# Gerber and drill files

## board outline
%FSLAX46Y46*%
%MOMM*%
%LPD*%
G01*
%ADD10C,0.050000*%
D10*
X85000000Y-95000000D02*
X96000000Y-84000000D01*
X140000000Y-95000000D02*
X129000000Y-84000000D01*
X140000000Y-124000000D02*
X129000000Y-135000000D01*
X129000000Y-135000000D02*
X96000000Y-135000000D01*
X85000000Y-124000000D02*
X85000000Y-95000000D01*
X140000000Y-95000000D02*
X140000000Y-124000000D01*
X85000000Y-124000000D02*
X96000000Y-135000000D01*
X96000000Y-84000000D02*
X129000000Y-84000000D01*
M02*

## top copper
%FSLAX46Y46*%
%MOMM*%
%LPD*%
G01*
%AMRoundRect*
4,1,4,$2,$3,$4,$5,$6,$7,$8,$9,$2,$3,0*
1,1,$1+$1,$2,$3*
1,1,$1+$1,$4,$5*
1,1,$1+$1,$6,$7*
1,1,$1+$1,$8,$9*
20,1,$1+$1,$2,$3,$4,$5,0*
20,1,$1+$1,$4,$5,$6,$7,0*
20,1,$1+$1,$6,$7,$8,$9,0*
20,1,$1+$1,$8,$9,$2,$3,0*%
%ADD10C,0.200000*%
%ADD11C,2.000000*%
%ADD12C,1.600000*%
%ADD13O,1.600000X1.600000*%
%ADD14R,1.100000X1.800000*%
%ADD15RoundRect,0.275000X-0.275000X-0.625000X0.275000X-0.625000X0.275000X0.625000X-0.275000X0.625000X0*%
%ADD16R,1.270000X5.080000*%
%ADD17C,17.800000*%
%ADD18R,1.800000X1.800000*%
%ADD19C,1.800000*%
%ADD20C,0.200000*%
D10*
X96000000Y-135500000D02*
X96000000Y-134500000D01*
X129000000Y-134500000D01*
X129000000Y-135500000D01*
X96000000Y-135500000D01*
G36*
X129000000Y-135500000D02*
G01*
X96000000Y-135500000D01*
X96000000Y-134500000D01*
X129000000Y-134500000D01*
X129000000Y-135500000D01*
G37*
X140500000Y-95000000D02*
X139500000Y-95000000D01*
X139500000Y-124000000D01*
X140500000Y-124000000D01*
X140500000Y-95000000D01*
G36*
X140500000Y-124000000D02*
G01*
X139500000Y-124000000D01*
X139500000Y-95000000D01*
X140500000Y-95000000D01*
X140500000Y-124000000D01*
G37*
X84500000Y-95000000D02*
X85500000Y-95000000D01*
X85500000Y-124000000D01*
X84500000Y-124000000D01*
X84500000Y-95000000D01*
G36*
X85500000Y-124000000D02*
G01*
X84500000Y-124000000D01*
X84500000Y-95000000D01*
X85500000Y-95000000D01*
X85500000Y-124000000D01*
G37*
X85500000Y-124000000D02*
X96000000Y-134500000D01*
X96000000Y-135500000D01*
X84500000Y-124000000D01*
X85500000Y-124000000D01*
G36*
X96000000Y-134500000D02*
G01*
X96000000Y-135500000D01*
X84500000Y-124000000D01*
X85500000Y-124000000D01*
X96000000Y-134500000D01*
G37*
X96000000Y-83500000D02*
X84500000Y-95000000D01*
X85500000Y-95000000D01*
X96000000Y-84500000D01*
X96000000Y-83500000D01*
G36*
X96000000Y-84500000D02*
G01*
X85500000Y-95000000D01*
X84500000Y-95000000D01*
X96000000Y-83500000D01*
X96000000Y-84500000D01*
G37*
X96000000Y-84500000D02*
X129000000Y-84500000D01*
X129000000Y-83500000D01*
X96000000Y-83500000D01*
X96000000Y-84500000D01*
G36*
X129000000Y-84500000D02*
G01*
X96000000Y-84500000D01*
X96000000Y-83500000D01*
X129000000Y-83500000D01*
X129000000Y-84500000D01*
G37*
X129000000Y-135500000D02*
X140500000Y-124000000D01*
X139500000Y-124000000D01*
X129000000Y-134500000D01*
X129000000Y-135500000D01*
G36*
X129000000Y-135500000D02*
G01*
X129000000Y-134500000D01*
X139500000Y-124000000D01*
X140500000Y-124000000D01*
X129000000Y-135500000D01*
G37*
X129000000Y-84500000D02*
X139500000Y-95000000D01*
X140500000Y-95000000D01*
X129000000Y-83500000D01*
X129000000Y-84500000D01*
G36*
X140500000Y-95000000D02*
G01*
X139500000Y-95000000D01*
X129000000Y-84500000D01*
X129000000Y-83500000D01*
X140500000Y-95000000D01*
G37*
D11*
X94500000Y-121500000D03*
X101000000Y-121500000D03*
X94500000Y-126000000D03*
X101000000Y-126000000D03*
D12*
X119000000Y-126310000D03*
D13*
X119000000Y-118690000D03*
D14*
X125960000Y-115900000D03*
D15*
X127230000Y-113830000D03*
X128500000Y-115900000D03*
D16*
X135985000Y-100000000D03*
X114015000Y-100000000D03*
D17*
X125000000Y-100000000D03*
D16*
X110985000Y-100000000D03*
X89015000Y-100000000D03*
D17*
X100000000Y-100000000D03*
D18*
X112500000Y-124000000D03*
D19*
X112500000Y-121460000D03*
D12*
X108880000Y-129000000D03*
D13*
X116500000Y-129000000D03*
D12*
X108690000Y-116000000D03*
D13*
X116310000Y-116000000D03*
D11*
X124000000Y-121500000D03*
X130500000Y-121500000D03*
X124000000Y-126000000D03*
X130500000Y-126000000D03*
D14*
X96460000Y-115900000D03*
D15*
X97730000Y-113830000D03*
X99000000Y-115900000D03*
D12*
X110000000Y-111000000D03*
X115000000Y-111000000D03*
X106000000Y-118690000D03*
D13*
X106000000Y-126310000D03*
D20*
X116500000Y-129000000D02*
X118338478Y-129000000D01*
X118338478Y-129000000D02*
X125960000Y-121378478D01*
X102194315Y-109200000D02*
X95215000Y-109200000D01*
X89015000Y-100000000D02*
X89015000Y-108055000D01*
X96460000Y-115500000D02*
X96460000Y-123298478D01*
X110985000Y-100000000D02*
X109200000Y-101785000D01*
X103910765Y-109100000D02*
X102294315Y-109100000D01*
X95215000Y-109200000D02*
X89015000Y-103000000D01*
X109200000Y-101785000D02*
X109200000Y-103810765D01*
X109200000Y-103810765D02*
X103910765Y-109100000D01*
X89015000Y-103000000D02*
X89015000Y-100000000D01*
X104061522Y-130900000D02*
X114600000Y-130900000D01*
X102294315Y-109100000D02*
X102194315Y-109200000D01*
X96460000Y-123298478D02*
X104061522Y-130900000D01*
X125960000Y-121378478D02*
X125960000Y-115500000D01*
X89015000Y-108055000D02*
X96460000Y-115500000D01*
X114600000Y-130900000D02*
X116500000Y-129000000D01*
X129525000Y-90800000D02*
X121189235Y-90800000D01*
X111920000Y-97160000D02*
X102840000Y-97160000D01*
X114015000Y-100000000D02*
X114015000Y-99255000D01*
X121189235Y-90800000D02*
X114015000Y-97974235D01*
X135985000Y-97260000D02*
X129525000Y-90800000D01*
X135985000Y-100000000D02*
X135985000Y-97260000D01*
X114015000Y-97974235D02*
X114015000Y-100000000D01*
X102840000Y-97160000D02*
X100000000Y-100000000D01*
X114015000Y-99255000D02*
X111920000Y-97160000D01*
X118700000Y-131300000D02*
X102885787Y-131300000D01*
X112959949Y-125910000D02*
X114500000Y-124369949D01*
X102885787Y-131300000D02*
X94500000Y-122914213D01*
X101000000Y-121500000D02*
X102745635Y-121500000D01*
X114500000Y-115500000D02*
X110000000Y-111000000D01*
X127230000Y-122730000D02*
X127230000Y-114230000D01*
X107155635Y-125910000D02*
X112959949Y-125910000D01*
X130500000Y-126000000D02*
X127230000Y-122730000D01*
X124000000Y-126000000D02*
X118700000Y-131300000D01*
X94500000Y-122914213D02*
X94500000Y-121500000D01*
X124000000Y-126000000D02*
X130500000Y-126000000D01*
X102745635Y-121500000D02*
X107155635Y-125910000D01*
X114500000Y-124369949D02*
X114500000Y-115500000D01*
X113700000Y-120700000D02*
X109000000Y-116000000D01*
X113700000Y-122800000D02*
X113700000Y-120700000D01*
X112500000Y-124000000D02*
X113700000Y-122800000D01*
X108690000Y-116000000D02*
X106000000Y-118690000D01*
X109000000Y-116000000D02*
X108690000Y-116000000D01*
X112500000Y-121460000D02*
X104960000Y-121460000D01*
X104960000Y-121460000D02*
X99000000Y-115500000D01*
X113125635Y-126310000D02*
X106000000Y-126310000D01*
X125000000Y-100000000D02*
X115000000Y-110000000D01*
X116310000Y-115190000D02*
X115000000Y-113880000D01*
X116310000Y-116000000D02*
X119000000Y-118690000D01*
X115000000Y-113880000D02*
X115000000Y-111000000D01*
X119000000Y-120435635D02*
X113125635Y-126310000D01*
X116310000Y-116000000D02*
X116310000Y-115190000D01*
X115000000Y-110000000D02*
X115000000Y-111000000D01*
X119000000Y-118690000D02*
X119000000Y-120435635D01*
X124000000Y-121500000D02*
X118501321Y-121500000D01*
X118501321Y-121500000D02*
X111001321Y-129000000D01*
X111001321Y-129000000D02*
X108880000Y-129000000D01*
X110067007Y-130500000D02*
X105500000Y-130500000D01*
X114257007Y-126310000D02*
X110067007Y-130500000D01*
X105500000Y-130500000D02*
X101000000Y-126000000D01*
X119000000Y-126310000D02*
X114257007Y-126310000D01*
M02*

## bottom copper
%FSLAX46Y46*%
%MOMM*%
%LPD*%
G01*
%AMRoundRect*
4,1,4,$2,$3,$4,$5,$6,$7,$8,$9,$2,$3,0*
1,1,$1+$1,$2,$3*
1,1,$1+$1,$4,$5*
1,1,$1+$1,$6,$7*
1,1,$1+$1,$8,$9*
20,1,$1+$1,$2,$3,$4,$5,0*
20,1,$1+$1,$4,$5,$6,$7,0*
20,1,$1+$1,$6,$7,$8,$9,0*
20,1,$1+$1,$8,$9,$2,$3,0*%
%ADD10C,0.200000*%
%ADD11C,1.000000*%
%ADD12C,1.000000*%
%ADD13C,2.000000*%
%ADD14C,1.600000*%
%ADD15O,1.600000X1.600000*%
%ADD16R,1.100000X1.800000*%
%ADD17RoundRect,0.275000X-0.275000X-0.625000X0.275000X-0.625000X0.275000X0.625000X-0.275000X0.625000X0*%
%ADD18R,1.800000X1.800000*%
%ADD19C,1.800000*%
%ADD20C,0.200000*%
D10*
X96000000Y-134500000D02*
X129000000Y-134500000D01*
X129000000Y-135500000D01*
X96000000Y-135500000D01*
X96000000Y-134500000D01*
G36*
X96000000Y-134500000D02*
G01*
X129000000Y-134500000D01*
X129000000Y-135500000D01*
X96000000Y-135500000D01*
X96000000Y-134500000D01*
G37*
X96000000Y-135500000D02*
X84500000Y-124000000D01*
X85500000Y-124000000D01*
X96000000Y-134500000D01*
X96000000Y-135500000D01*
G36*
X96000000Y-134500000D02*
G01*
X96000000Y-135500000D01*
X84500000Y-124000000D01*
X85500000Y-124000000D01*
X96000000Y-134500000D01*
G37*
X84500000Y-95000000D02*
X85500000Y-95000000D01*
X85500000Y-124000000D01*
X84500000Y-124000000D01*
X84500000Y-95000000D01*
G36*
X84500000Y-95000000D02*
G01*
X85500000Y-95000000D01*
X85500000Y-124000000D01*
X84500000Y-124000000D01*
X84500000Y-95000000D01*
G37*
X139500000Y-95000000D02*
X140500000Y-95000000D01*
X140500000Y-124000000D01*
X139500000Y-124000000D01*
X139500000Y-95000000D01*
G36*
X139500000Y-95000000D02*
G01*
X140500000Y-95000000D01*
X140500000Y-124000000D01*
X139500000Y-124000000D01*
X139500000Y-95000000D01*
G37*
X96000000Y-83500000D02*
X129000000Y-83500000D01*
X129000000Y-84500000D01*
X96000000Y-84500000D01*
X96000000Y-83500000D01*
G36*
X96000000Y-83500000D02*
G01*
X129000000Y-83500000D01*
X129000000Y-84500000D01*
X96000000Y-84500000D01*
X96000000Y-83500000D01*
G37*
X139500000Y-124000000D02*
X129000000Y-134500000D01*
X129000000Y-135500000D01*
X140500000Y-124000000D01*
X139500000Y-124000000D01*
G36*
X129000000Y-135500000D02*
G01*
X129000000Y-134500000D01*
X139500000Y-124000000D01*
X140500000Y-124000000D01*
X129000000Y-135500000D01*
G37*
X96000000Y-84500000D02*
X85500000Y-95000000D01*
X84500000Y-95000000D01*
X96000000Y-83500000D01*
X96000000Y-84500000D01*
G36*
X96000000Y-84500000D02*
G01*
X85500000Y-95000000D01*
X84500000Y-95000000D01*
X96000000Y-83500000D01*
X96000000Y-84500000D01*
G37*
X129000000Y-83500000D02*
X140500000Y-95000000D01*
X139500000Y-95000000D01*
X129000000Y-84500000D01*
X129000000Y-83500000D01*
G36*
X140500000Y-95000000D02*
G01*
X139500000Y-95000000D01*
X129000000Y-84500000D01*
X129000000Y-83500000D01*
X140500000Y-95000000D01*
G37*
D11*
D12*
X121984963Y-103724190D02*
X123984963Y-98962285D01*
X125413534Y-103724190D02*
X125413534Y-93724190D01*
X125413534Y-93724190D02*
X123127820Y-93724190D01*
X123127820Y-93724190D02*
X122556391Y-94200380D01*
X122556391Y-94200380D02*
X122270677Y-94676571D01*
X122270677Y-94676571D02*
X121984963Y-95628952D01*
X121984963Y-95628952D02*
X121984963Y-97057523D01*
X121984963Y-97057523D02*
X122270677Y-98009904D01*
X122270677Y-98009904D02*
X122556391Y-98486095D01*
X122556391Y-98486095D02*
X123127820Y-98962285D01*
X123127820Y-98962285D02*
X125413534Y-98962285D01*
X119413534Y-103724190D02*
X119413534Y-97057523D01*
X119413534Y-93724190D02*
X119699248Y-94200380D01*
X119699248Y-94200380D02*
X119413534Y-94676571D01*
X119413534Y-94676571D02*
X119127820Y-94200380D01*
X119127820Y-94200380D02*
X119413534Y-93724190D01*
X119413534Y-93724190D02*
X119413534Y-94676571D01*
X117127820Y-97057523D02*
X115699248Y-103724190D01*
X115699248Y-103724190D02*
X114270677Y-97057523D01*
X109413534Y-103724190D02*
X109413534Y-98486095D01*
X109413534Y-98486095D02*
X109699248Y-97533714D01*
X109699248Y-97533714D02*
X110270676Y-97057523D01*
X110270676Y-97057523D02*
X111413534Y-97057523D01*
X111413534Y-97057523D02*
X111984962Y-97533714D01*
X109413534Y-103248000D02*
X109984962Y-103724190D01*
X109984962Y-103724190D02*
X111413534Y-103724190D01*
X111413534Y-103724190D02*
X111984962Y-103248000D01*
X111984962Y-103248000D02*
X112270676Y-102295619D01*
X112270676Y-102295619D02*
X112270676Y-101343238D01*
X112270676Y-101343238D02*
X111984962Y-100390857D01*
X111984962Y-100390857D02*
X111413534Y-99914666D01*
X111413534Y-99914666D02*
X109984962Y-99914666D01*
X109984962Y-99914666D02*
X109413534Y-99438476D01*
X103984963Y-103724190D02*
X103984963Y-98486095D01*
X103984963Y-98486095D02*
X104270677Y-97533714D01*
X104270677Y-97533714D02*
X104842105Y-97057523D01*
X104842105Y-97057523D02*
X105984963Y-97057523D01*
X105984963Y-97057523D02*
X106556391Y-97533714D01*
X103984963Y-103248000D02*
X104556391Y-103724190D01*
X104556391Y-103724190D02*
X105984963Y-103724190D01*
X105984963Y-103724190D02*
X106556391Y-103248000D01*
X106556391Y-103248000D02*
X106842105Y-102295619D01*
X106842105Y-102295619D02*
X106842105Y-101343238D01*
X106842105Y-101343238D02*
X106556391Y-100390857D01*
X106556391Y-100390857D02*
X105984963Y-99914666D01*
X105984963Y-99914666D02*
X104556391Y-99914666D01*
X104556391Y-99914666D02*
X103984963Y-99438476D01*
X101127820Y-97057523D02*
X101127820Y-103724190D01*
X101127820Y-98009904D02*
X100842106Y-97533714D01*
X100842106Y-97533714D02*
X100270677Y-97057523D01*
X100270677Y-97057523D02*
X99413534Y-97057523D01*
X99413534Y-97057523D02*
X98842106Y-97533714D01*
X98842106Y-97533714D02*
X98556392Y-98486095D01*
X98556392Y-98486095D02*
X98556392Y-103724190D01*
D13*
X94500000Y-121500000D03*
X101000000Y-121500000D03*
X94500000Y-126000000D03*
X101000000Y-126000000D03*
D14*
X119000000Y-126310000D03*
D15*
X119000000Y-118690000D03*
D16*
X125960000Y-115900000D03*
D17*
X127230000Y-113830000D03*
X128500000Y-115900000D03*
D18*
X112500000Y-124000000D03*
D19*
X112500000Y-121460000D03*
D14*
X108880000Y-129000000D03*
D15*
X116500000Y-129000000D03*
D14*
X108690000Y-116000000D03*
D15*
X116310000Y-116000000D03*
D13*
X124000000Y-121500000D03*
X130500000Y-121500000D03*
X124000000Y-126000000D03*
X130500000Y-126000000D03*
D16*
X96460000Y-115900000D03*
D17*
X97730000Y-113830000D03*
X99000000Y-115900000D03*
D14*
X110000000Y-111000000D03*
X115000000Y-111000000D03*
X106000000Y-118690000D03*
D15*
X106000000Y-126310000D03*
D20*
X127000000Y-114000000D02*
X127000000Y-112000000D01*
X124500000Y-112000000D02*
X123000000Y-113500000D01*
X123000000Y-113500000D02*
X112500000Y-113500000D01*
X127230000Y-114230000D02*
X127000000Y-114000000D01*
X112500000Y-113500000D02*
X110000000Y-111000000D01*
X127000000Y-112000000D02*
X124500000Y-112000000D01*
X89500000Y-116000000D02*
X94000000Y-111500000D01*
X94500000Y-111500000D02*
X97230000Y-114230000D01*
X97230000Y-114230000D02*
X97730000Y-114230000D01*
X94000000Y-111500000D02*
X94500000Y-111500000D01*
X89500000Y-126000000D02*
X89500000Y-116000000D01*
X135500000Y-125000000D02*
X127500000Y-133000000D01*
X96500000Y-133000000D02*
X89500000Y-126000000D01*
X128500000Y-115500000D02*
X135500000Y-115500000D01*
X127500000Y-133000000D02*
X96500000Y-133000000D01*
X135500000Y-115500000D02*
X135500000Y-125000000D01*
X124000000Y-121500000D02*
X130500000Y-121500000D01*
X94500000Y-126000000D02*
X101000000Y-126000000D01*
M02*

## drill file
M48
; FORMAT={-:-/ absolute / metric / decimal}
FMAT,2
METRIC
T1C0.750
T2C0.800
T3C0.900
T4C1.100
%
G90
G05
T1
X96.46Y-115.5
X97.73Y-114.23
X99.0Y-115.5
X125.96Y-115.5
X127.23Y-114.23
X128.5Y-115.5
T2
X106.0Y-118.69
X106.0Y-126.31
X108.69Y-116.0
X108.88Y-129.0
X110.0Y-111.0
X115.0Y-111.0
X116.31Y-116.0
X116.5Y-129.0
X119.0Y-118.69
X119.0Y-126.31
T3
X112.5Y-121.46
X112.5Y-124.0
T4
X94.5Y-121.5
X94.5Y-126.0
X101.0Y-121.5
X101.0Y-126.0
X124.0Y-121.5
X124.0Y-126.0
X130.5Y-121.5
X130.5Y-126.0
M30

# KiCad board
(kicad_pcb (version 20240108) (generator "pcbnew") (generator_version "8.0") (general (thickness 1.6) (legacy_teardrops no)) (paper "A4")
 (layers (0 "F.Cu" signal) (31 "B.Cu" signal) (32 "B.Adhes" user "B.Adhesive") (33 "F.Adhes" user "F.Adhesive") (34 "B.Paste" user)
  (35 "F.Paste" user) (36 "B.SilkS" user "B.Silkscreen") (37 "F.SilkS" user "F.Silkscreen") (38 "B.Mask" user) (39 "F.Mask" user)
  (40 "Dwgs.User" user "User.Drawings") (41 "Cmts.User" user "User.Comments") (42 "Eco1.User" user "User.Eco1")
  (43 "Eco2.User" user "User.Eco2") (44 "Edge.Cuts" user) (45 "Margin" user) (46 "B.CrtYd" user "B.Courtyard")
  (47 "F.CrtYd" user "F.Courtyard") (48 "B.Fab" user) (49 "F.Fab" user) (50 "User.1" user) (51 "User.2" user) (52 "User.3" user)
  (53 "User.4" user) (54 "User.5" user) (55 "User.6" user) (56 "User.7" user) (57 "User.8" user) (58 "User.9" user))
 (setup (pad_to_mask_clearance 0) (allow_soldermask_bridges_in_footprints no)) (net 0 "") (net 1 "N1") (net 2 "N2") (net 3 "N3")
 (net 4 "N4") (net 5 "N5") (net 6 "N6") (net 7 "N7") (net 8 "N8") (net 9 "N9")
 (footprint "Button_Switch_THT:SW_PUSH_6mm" (layer "F.Cu") (at 94.5 121.5)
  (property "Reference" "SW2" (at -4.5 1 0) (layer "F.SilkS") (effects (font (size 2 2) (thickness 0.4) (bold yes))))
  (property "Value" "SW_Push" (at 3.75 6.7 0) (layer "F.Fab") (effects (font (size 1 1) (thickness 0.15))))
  (pad "1" thru_hole circle (at 0 0 90) (size 2 2) (drill 1.1) (layers "*.Cu" "*.Mask") (remove_unused_layers no) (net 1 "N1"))
  (pad "1" thru_hole circle (at 6.5 0 90) (size 2 2) (drill 1.1) (layers "*.Cu" "*.Mask") (remove_unused_layers no) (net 1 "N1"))
  (pad "2" thru_hole circle (at 0 4.5 90) (size 2 2) (drill 1.1) (layers "*.Cu" "*.Mask") (remove_unused_layers no) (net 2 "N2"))
  (pad "2" thru_hole circle (at 6.5 4.5 90) (size 2 2) (drill 1.1) (layers "*.Cu" "*.Mask") (remove_unused_layers no) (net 2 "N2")))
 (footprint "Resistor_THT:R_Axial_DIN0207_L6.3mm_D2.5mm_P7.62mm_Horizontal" (layer "F.Cu") (at 119 126.31 90)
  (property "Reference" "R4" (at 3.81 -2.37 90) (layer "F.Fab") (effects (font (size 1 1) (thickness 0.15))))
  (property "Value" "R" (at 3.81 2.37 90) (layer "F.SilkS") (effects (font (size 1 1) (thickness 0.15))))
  (pad "1" thru_hole circle (at 0 0 90) (size 1.6 1.6) (drill 0.8) (layers "*.Cu" "*.Mask") (remove_unused_layers no) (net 2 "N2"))
  (pad "2" thru_hole oval (at 7.62 0 90) (size 1.6 1.6) (drill 0.8) (layers "*.Cu" "*.Mask") (remove_unused_layers no) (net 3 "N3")))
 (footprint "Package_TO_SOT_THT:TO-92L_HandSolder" (layer "F.Cu") (at 125.96 115.5)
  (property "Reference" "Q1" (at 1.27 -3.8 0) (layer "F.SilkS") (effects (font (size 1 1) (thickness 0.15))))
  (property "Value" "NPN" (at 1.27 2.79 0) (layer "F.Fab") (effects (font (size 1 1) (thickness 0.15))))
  (pad "1" thru_hole rect (at 0 0) (size 1.1 1.8) (drill 0.75 (offset 0 0.4)) (layers "*.Cu" "*.Mask") (remove_unused_layers no)
   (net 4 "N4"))
  (pad "2" thru_hole roundrect (at 1.27 -1.27) (size 1.1 1.8) (drill 0.75 (offset 0 -0.4)) (layers "*.Cu" "*.Mask")
   (remove_unused_layers no) (roundrect_rratio 0.25) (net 1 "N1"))
  (pad "3" thru_hole roundrect (at 2.54 0) (size 1.1 1.8) (drill 0.75 (offset 0 0.4)) (layers "*.Cu" "*.Mask") (remove_unused_layers no)
   (roundrect_rratio 0.25) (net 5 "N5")))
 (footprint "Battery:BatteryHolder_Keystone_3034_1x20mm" (layer "F.Cu") (at 125 100 180)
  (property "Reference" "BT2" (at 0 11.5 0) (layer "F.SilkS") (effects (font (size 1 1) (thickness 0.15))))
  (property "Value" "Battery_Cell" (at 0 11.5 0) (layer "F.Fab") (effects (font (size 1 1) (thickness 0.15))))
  (pad "1" smd rect (at -10.985 0 180) (size 1.27 5.08) (layers "F.Cu" "F.Paste" "F.Mask") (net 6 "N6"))
  (pad "1" smd rect (at 10.985 0 180) (size 1.27 5.08) (layers "F.Cu" "F.Paste" "F.Mask") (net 6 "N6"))
  (pad "2" smd circle (at 0 0 180) (size 17.8 17.8) (layers "F.Cu" "F.Mask") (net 3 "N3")))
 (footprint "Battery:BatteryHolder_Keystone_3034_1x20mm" (layer "F.Cu") (at 100 100 180)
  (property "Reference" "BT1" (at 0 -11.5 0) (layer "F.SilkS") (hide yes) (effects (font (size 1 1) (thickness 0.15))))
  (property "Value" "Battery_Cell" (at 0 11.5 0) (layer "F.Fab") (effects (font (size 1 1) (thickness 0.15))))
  (pad "1" smd rect (at -10.985 0 180) (size 1.27 5.08) (layers "F.Cu" "F.Paste" "F.Mask") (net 4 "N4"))
  (pad "1" smd rect (at 10.985 0 180) (size 1.27 5.08) (layers "F.Cu" "F.Paste" "F.Mask") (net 4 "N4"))
  (pad "2" smd circle (at 0 0 180) (size 17.8 17.8) (layers "F.Cu" "F.Mask") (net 6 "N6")))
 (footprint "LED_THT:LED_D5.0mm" (layer "F.Cu") (at 112.5 124 90)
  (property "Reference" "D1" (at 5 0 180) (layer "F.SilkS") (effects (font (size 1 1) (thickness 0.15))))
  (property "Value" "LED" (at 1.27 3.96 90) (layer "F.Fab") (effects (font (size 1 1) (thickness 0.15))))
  (pad "1" thru_hole rect (at 0 0 90) (size 1.8 1.8) (drill 0.9) (layers "*.Cu" "*.Mask") (remove_unused_layers no) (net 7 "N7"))
  (pad "2" thru_hole circle (at 2.54 0 90) (size 1.8 1.8) (drill 0.9) (layers "*.Cu" "*.Mask") (remove_unused_layers no) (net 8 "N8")))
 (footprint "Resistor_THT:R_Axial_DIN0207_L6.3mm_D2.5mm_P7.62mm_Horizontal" (layer "F.Cu") (at 108.88 129)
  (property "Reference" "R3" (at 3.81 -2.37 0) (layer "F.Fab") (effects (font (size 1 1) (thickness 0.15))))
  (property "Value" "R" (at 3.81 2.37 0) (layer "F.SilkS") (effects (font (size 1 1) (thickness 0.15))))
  (pad "1" thru_hole circle (at 0 0) (size 1.6 1.6) (drill 0.8) (layers "*.Cu" "*.Mask") (remove_unused_layers no) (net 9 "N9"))
  (pad "2" thru_hole oval (at 7.62 0) (size 1.6 1.6) (drill 0.8) (layers "*.Cu" "*.Mask") (remove_unused_layers no) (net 4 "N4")))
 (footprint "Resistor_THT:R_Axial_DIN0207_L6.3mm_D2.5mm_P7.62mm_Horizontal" (layer "F.Cu") (at 108.69 116)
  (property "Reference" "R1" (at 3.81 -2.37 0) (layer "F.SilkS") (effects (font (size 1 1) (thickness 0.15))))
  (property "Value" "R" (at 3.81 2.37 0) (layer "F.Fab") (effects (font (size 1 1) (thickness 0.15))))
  (pad "1" thru_hole circle (at 0 0) (size 1.6 1.6) (drill 0.8) (layers "*.Cu" "*.Mask") (remove_unused_layers no) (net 7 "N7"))
  (pad "2" thru_hole oval (at 7.62 0) (size 1.6 1.6) (drill 0.8) (layers "*.Cu" "*.Mask") (remove_unused_layers no) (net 3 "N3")))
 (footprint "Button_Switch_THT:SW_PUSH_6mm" (layer "F.Cu") (at 124 121.5)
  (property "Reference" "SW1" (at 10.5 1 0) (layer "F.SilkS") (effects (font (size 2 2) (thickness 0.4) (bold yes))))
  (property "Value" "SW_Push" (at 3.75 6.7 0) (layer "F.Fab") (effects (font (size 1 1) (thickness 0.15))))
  (pad "1" thru_hole circle (at 0 0 90) (size 2 2) (drill 1.1) (layers "*.Cu" "*.Mask") (remove_unused_layers no) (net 9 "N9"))
  (pad "1" thru_hole circle (at 6.5 0 90) (size 2 2) (drill 1.1) (layers "*.Cu" "*.Mask") (remove_unused_layers no) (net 9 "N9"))
  (pad "2" thru_hole circle (at 0 4.5 90) (size 2 2) (drill 1.1) (layers "*.Cu" "*.Mask") (remove_unused_layers no) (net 1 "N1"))
  (pad "2" thru_hole circle (at 6.5 4.5 90) (size 2 2) (drill 1.1) (layers "*.Cu" "*.Mask") (remove_unused_layers no) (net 1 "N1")))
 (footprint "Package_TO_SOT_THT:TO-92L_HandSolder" (layer "F.Cu") (at 96.46 115.5)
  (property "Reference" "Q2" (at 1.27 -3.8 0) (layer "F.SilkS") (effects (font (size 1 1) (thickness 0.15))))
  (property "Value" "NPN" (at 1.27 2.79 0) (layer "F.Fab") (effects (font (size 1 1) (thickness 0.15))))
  (pad "1" thru_hole rect (at 0 0) (size 1.1 1.8) (drill 0.75 (offset 0 0.4)) (layers "*.Cu" "*.Mask") (remove_unused_layers no)
   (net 4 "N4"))
  (pad "2" thru_hole roundrect (at 1.27 -1.27) (size 1.1 1.8) (drill 0.75 (offset 0 -0.4)) (layers "*.Cu" "*.Mask")
   (remove_unused_layers no) (roundrect_rratio 0.25) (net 5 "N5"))
  (pad "3" thru_hole roundrect (at 2.54 0) (size 1.1 1.8) (drill 0.75 (offset 0 0.4)) (layers "*.Cu" "*.Mask") (remove_unused_layers no)
   (roundrect_rratio 0.25) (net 8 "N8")))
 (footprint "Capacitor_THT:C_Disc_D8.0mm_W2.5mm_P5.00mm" (layer "F.Cu") (at 110 111)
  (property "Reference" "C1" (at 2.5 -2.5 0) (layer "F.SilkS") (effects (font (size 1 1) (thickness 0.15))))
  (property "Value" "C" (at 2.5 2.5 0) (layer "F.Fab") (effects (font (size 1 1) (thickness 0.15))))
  (pad "1" thru_hole circle (at 0 0) (size 1.6 1.6) (drill 0.8) (layers "*.Cu" "*.Mask") (remove_unused_layers no) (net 1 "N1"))
  (pad "2" thru_hole circle (at 5 0) (size 1.6 1.6) (drill 0.8) (layers "*.Cu" "*.Mask") (remove_unused_layers no) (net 3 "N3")))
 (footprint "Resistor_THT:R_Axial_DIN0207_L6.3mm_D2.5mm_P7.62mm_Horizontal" (layer "F.Cu") (at 106 118.69 -90)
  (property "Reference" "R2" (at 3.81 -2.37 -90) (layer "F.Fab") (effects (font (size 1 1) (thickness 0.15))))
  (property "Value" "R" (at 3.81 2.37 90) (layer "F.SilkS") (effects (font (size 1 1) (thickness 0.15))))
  (pad "1" thru_hole circle (at 0 0 270) (size 1.6 1.6) (drill 0.8) (layers "*.Cu" "*.Mask") (remove_unused_layers no) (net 7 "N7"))
  (pad "2" thru_hole oval (at 7.62 0 270) (size 1.6 1.6) (drill 0.8) (layers "*.Cu" "*.Mask") (remove_unused_layers no) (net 3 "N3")))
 (gr_poly (pts (xy 96 135.5) (xy 96 134.5) (xy 129 134.5) (xy 129 135.5)) (stroke (width 0.2) (type solid)) (fill solid) (layer "F.Cu"))
 (gr_poly (pts (xy 140.5 95) (xy 139.5 95) (xy 139.5 124) (xy 140.5 124)) (stroke (width 0.2) (type solid)) (fill solid) (layer "F.Cu"))
 (gr_poly (pts (xy 84.5 95) (xy 85.5 95) (xy 85.5 124) (xy 84.5 124)) (stroke (width 0.2) (type solid)) (fill solid) (layer "F.Cu"))
 (gr_poly (pts (xy 85.5 124) (xy 96 134.5) (xy 96 135.5) (xy 84.5 124)) (stroke (width 0.2) (type solid)) (fill solid) (layer "F.Cu"))
 (gr_poly (pts (xy 96 83.5) (xy 84.5 95) (xy 85.5 95) (xy 96 84.5)) (stroke (width 0.2) (type solid)) (fill solid) (layer "F.Cu"))
 (gr_poly (pts (xy 96 84.5) (xy 129 84.5) (xy 129 83.5) (xy 96 83.5)) (stroke (width 0.2) (type solid)) (fill solid) (layer "F.Cu"))
 (gr_poly (pts (xy 129 135.5) (xy 140.5 124) (xy 139.5 124) (xy 129 134.5)) (stroke (width 0.2) (type solid)) (fill solid) (layer "F.Cu"))
 (gr_poly (pts (xy 129 84.5) (xy 139.5 95) (xy 140.5 95) (xy 129 83.5)) (stroke (width 0.2) (type solid)) (fill solid) (layer "F.Cu"))
 (gr_rect (start 96 134.5) (end 129 135.5) (stroke (width 0.2) (type solid)) (fill solid) (layer "B.Cu"))
 (gr_poly (pts (xy 96 135.5) (xy 84.5 124) (xy 85.5 124) (xy 96 134.5)) (stroke (width 0.2) (type solid)) (fill solid) (layer "B.Cu"))
 (gr_rect (start 84.5 95) (end 85.5 124) (stroke (width 0.2) (type solid)) (fill solid) (layer "B.Cu"))
 (gr_rect (start 139.5 95) (end 140.5 124) (stroke (width 0.2) (type solid)) (fill solid) (layer "B.Cu"))
 (gr_rect (start 96 83.5) (end 129 84.5) (stroke (width 0.2) (type solid)) (fill solid) (layer "B.Cu"))
 (gr_poly (pts (xy 139.5 124) (xy 129 134.5) (xy 129 135.5) (xy 140.5 124)) (stroke (width 0.2) (type solid)) (fill solid) (layer "B.Cu"))
 (gr_poly (pts (xy 96 84.5) (xy 85.5 95) (xy 84.5 95) (xy 96 83.5)) (stroke (width 0.2) (type solid)) (fill solid) (layer "B.Cu"))
 (gr_poly (pts (xy 129 83.5) (xy 140.5 95) (xy 139.5 95) (xy 129 84.5)) (stroke (width 0.2) (type solid)) (fill solid) (layer "B.Cu"))
 (gr_line (start 85 95) (end 96 84) (stroke (width 0.05) (type default)) (layer "Edge.Cuts"))
 (gr_line (start 140 95) (end 129 84) (stroke (width 0.05) (type default)) (layer "Edge.Cuts"))
 (gr_line (start 140 124) (end 129 135) (stroke (width 0.05) (type default)) (layer "Edge.Cuts"))
 (gr_line (start 129 135) (end 96 135) (stroke (width 0.05) (type default)) (layer "Edge.Cuts"))
 (gr_line (start 85 124) (end 85 95) (stroke (width 0.05) (type default)) (layer "Edge.Cuts"))
 (gr_line (start 140 95) (end 140 124) (stroke (width 0.05) (type default)) (layer "Edge.Cuts"))
 (gr_line (start 85 124) (end 96 135) (stroke (width 0.05) (type default)) (layer "Edge.Cuts"))
 (gr_line (start 96 84) (end 129 84) (stroke (width 0.05) (type default)) (layer "Edge.Cuts"))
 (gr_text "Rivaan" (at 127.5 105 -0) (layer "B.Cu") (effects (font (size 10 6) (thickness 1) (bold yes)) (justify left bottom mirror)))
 (segment (start 116.5 129) (end 118.338478 129) (width 0.2) (layer "F.Cu") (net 4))
 (segment (start 118.338478 129) (end 125.96 121.378478) (width 0.2) (layer "F.Cu") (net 4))
 (segment (start 102.194315 109.2) (end 95.215 109.2) (width 0.2) (layer "F.Cu") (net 4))
 (segment (start 89.015 100) (end 89.015 108.055) (width 0.2) (layer "F.Cu") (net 4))
 (segment (start 96.46 115.5) (end 96.46 123.298478) (width 0.2) (layer "F.Cu") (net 4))
 (segment (start 110.985 100) (end 109.2 101.785) (width 0.2) (layer "F.Cu") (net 4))
 (segment (start 103.910765 109.1) (end 102.294315 109.1) (width 0.2) (layer "F.Cu") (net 4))
 (segment (start 95.215 109.2) (end 89.015 103) (width 0.2) (layer "F.Cu") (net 4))
 (segment (start 109.2 101.785) (end 109.2 103.810765) (width 0.2) (layer "F.Cu") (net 4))
 (segment (start 109.2 103.810765) (end 103.910765 109.1) (width 0.2) (layer "F.Cu") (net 4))
 (segment (start 89.015 103) (end 89.015 100) (width 0.2) (layer "F.Cu") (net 4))
 (segment (start 104.061522 130.9) (end 114.6 130.9) (width 0.2) (layer "F.Cu") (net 4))
 (segment (start 102.294315 109.1) (end 102.194315 109.2) (width 0.2) (layer "F.Cu") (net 4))
 (segment (start 96.46 123.298478) (end 104.061522 130.9) (width 0.2) (layer "F.Cu") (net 4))
 (segment (start 125.96 121.378478) (end 125.96 115.5) (width 0.2) (layer "F.Cu") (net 4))
 (segment (start 89.015 108.055) (end 96.46 115.5) (width 0.2) (layer "F.Cu") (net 4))
 (segment (start 114.6 130.9) (end 116.5 129) (width 0.2) (layer "F.Cu") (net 4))
 (segment (start 129.525 90.8) (end 121.189235 90.8) (width 0.2) (layer "F.Cu") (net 6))
 (segment (start 111.92 97.16) (end 102.84 97.16) (width 0.2) (layer "F.Cu") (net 6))
 (segment (start 114.015 100) (end 114.015 99.255) (width 0.2) (layer "F.Cu") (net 6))
 (segment (start 121.189235 90.8) (end 114.015 97.974235) (width 0.2) (layer "F.Cu") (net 6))
 (segment (start 135.985 97.26) (end 129.525 90.8) (width 0.2) (layer "F.Cu") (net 6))
 (segment (start 135.985 100) (end 135.985 97.26) (width 0.2) (layer "F.Cu") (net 6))
 (segment (start 114.015 97.974235) (end 114.015 100) (width 0.2) (layer "F.Cu") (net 6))
 (segment (start 102.84 97.16) (end 100 100) (width 0.2) (layer "F.Cu") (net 6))
 (segment (start 114.015 99.255) (end 111.92 97.16) (width 0.2) (layer "F.Cu") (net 6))
 (segment (start 118.7 131.3) (end 102.885787 131.3) (width 0.2) (layer "F.Cu") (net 1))
 (segment (start 112.959949 125.91) (end 114.5 124.369949) (width 0.2) (layer "F.Cu") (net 1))
 (segment (start 102.885787 131.3) (end 94.5 122.914213) (width 0.2) (layer "F.Cu") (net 1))
 (segment (start 101 121.5) (end 102.745635 121.5) (width 0.2) (layer "F.Cu") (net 1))
 (segment (start 114.5 115.5) (end 110 111) (width 0.2) (layer "F.Cu") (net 1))
 (segment (start 127.23 122.73) (end 127.23 114.23) (width 0.2) (layer "F.Cu") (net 1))
 (segment (start 107.155635 125.91) (end 112.959949 125.91) (width 0.2) (layer "F.Cu") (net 1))
 (segment (start 130.5 126) (end 127.23 122.73) (width 0.2) (layer "F.Cu") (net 1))
 (segment (start 124 126) (end 118.7 131.3) (width 0.2) (layer "F.Cu") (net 1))
 (segment (start 94.5 122.914213) (end 94.5 121.5) (width 0.2) (layer "F.Cu") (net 1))
 (segment (start 124 126) (end 130.5 126) (width 0.2) (layer "F.Cu") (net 1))
 (segment (start 102.745635 121.5) (end 107.155635 125.91) (width 0.2) (layer "F.Cu") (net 1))
 (segment (start 114.5 124.369949) (end 114.5 115.5) (width 0.2) (layer "F.Cu") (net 1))
 (segment (start 127 114) (end 127 112) (width 0.2) (layer "B.Cu") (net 1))
 (segment (start 124.5 112) (end 123 113.5) (width 0.2) (layer "B.Cu") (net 1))
 (segment (start 123 113.5) (end 112.5 113.5) (width 0.2) (layer "B.Cu") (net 1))
 (segment (start 127.23 114.23) (end 127 114) (width 0.2) (layer "B.Cu") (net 1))
 (segment (start 112.5 113.5) (end 110 111) (width 0.2) (layer "B.Cu") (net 1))
 (segment (start 127 112) (end 124.5 112) (width 0.2) (layer "B.Cu") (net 1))
 (segment (start 113.7 120.7) (end 109 116) (width 0.2) (layer "F.Cu") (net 7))
 (segment (start 113.7 122.8) (end 113.7 120.7) (width 0.2) (layer "F.Cu") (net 7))
 (segment (start 112.5 124) (end 113.7 122.8) (width 0.2) (layer "F.Cu") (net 7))
 (segment (start 108.69 116) (end 106 118.69) (width 0.2) (layer "F.Cu") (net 7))
 (segment (start 109 116) (end 108.69 116) (width 0.2) (layer "F.Cu") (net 7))
 (segment (start 112.5 121.46) (end 104.96 121.46) (width 0.2) (layer "F.Cu") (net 8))
 (segment (start 104.96 121.46) (end 99 115.5) (width 0.2) (layer "F.Cu") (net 8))
 (segment (start 89.5 116) (end 94 111.5) (width 0.2) (layer "B.Cu") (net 5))
 (segment (start 94.5 111.5) (end 97.23 114.23) (width 0.2) (layer "B.Cu") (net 5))
 (segment (start 97.23 114.23) (end 97.73 114.23) (width 0.2) (layer "B.Cu") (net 5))
 (segment (start 94 111.5) (end 94.5 111.5) (width 0.2) (layer "B.Cu") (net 5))
 (segment (start 89.5 126) (end 89.5 116) (width 0.2) (layer "B.Cu") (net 5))
 (segment (start 135.5 125) (end 127.5 133) (width 0.2) (layer "B.Cu") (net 5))
 (segment (start 96.5 133) (end 89.5 126) (width 0.2) (layer "B.Cu") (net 5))
 (segment (start 128.5 115.5) (end 135.5 115.5) (width 0.2) (layer "B.Cu") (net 5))
 (segment (start 127.5 133) (end 96.5 133) (width 0.2) (layer "B.Cu") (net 5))
 (segment (start 135.5 115.5) (end 135.5 125) (width 0.2) (layer "B.Cu") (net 5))
 (segment (start 113.125635 126.31) (end 106 126.31) (width 0.2) (layer "F.Cu") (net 3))
 (segment (start 125 100) (end 115 110) (width 0.2) (layer "F.Cu") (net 3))
 (segment (start 116.31 115.19) (end 115 113.88) (width 0.2) (layer "F.Cu") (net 3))
 (segment (start 116.31 116) (end 119 118.69) (width 0.2) (layer "F.Cu") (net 3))
 (segment (start 115 113.88) (end 115 111) (width 0.2) (layer "F.Cu") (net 3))
 (segment (start 119 120.435635) (end 113.125635 126.31) (width 0.2) (layer "F.Cu") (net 3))
 (segment (start 116.31 116) (end 116.31 115.19) (width 0.2) (layer "F.Cu") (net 3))
 (segment (start 115 110) (end 115 111) (width 0.2) (layer "F.Cu") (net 3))
 (segment (start 119 118.69) (end 119 120.435635) (width 0.2) (layer "F.Cu") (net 3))
 (segment (start 124 121.5) (end 118.501321 121.5) (width 0.2) (layer "F.Cu") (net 9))
 (segment (start 118.501321 121.5) (end 111.001321 129) (width 0.2) (layer "F.Cu") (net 9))
 (segment (start 111.001321 129) (end 108.88 129) (width 0.2) (layer "F.Cu") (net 9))
 (segment (start 124 121.5) (end 130.5 121.5) (width 0.2) (layer "B.Cu") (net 9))
 (segment (start 110.067007 130.5) (end 105.5 130.5) (width 0.2) (layer "F.Cu") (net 2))
 (segment (start 114.257007 126.31) (end 110.067007 130.5) (width 0.2) (layer "F.Cu") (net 2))
 (segment (start 105.5 130.5) (end 101 126) (width 0.2) (layer "F.Cu") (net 2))
 (segment (start 119 126.31) (end 114.257007 126.31) (width 0.2) (layer "F.Cu") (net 2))
 (segment (start 94.5 126) (end 101 126) (width 0.2) (layer "B.Cu") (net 2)))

